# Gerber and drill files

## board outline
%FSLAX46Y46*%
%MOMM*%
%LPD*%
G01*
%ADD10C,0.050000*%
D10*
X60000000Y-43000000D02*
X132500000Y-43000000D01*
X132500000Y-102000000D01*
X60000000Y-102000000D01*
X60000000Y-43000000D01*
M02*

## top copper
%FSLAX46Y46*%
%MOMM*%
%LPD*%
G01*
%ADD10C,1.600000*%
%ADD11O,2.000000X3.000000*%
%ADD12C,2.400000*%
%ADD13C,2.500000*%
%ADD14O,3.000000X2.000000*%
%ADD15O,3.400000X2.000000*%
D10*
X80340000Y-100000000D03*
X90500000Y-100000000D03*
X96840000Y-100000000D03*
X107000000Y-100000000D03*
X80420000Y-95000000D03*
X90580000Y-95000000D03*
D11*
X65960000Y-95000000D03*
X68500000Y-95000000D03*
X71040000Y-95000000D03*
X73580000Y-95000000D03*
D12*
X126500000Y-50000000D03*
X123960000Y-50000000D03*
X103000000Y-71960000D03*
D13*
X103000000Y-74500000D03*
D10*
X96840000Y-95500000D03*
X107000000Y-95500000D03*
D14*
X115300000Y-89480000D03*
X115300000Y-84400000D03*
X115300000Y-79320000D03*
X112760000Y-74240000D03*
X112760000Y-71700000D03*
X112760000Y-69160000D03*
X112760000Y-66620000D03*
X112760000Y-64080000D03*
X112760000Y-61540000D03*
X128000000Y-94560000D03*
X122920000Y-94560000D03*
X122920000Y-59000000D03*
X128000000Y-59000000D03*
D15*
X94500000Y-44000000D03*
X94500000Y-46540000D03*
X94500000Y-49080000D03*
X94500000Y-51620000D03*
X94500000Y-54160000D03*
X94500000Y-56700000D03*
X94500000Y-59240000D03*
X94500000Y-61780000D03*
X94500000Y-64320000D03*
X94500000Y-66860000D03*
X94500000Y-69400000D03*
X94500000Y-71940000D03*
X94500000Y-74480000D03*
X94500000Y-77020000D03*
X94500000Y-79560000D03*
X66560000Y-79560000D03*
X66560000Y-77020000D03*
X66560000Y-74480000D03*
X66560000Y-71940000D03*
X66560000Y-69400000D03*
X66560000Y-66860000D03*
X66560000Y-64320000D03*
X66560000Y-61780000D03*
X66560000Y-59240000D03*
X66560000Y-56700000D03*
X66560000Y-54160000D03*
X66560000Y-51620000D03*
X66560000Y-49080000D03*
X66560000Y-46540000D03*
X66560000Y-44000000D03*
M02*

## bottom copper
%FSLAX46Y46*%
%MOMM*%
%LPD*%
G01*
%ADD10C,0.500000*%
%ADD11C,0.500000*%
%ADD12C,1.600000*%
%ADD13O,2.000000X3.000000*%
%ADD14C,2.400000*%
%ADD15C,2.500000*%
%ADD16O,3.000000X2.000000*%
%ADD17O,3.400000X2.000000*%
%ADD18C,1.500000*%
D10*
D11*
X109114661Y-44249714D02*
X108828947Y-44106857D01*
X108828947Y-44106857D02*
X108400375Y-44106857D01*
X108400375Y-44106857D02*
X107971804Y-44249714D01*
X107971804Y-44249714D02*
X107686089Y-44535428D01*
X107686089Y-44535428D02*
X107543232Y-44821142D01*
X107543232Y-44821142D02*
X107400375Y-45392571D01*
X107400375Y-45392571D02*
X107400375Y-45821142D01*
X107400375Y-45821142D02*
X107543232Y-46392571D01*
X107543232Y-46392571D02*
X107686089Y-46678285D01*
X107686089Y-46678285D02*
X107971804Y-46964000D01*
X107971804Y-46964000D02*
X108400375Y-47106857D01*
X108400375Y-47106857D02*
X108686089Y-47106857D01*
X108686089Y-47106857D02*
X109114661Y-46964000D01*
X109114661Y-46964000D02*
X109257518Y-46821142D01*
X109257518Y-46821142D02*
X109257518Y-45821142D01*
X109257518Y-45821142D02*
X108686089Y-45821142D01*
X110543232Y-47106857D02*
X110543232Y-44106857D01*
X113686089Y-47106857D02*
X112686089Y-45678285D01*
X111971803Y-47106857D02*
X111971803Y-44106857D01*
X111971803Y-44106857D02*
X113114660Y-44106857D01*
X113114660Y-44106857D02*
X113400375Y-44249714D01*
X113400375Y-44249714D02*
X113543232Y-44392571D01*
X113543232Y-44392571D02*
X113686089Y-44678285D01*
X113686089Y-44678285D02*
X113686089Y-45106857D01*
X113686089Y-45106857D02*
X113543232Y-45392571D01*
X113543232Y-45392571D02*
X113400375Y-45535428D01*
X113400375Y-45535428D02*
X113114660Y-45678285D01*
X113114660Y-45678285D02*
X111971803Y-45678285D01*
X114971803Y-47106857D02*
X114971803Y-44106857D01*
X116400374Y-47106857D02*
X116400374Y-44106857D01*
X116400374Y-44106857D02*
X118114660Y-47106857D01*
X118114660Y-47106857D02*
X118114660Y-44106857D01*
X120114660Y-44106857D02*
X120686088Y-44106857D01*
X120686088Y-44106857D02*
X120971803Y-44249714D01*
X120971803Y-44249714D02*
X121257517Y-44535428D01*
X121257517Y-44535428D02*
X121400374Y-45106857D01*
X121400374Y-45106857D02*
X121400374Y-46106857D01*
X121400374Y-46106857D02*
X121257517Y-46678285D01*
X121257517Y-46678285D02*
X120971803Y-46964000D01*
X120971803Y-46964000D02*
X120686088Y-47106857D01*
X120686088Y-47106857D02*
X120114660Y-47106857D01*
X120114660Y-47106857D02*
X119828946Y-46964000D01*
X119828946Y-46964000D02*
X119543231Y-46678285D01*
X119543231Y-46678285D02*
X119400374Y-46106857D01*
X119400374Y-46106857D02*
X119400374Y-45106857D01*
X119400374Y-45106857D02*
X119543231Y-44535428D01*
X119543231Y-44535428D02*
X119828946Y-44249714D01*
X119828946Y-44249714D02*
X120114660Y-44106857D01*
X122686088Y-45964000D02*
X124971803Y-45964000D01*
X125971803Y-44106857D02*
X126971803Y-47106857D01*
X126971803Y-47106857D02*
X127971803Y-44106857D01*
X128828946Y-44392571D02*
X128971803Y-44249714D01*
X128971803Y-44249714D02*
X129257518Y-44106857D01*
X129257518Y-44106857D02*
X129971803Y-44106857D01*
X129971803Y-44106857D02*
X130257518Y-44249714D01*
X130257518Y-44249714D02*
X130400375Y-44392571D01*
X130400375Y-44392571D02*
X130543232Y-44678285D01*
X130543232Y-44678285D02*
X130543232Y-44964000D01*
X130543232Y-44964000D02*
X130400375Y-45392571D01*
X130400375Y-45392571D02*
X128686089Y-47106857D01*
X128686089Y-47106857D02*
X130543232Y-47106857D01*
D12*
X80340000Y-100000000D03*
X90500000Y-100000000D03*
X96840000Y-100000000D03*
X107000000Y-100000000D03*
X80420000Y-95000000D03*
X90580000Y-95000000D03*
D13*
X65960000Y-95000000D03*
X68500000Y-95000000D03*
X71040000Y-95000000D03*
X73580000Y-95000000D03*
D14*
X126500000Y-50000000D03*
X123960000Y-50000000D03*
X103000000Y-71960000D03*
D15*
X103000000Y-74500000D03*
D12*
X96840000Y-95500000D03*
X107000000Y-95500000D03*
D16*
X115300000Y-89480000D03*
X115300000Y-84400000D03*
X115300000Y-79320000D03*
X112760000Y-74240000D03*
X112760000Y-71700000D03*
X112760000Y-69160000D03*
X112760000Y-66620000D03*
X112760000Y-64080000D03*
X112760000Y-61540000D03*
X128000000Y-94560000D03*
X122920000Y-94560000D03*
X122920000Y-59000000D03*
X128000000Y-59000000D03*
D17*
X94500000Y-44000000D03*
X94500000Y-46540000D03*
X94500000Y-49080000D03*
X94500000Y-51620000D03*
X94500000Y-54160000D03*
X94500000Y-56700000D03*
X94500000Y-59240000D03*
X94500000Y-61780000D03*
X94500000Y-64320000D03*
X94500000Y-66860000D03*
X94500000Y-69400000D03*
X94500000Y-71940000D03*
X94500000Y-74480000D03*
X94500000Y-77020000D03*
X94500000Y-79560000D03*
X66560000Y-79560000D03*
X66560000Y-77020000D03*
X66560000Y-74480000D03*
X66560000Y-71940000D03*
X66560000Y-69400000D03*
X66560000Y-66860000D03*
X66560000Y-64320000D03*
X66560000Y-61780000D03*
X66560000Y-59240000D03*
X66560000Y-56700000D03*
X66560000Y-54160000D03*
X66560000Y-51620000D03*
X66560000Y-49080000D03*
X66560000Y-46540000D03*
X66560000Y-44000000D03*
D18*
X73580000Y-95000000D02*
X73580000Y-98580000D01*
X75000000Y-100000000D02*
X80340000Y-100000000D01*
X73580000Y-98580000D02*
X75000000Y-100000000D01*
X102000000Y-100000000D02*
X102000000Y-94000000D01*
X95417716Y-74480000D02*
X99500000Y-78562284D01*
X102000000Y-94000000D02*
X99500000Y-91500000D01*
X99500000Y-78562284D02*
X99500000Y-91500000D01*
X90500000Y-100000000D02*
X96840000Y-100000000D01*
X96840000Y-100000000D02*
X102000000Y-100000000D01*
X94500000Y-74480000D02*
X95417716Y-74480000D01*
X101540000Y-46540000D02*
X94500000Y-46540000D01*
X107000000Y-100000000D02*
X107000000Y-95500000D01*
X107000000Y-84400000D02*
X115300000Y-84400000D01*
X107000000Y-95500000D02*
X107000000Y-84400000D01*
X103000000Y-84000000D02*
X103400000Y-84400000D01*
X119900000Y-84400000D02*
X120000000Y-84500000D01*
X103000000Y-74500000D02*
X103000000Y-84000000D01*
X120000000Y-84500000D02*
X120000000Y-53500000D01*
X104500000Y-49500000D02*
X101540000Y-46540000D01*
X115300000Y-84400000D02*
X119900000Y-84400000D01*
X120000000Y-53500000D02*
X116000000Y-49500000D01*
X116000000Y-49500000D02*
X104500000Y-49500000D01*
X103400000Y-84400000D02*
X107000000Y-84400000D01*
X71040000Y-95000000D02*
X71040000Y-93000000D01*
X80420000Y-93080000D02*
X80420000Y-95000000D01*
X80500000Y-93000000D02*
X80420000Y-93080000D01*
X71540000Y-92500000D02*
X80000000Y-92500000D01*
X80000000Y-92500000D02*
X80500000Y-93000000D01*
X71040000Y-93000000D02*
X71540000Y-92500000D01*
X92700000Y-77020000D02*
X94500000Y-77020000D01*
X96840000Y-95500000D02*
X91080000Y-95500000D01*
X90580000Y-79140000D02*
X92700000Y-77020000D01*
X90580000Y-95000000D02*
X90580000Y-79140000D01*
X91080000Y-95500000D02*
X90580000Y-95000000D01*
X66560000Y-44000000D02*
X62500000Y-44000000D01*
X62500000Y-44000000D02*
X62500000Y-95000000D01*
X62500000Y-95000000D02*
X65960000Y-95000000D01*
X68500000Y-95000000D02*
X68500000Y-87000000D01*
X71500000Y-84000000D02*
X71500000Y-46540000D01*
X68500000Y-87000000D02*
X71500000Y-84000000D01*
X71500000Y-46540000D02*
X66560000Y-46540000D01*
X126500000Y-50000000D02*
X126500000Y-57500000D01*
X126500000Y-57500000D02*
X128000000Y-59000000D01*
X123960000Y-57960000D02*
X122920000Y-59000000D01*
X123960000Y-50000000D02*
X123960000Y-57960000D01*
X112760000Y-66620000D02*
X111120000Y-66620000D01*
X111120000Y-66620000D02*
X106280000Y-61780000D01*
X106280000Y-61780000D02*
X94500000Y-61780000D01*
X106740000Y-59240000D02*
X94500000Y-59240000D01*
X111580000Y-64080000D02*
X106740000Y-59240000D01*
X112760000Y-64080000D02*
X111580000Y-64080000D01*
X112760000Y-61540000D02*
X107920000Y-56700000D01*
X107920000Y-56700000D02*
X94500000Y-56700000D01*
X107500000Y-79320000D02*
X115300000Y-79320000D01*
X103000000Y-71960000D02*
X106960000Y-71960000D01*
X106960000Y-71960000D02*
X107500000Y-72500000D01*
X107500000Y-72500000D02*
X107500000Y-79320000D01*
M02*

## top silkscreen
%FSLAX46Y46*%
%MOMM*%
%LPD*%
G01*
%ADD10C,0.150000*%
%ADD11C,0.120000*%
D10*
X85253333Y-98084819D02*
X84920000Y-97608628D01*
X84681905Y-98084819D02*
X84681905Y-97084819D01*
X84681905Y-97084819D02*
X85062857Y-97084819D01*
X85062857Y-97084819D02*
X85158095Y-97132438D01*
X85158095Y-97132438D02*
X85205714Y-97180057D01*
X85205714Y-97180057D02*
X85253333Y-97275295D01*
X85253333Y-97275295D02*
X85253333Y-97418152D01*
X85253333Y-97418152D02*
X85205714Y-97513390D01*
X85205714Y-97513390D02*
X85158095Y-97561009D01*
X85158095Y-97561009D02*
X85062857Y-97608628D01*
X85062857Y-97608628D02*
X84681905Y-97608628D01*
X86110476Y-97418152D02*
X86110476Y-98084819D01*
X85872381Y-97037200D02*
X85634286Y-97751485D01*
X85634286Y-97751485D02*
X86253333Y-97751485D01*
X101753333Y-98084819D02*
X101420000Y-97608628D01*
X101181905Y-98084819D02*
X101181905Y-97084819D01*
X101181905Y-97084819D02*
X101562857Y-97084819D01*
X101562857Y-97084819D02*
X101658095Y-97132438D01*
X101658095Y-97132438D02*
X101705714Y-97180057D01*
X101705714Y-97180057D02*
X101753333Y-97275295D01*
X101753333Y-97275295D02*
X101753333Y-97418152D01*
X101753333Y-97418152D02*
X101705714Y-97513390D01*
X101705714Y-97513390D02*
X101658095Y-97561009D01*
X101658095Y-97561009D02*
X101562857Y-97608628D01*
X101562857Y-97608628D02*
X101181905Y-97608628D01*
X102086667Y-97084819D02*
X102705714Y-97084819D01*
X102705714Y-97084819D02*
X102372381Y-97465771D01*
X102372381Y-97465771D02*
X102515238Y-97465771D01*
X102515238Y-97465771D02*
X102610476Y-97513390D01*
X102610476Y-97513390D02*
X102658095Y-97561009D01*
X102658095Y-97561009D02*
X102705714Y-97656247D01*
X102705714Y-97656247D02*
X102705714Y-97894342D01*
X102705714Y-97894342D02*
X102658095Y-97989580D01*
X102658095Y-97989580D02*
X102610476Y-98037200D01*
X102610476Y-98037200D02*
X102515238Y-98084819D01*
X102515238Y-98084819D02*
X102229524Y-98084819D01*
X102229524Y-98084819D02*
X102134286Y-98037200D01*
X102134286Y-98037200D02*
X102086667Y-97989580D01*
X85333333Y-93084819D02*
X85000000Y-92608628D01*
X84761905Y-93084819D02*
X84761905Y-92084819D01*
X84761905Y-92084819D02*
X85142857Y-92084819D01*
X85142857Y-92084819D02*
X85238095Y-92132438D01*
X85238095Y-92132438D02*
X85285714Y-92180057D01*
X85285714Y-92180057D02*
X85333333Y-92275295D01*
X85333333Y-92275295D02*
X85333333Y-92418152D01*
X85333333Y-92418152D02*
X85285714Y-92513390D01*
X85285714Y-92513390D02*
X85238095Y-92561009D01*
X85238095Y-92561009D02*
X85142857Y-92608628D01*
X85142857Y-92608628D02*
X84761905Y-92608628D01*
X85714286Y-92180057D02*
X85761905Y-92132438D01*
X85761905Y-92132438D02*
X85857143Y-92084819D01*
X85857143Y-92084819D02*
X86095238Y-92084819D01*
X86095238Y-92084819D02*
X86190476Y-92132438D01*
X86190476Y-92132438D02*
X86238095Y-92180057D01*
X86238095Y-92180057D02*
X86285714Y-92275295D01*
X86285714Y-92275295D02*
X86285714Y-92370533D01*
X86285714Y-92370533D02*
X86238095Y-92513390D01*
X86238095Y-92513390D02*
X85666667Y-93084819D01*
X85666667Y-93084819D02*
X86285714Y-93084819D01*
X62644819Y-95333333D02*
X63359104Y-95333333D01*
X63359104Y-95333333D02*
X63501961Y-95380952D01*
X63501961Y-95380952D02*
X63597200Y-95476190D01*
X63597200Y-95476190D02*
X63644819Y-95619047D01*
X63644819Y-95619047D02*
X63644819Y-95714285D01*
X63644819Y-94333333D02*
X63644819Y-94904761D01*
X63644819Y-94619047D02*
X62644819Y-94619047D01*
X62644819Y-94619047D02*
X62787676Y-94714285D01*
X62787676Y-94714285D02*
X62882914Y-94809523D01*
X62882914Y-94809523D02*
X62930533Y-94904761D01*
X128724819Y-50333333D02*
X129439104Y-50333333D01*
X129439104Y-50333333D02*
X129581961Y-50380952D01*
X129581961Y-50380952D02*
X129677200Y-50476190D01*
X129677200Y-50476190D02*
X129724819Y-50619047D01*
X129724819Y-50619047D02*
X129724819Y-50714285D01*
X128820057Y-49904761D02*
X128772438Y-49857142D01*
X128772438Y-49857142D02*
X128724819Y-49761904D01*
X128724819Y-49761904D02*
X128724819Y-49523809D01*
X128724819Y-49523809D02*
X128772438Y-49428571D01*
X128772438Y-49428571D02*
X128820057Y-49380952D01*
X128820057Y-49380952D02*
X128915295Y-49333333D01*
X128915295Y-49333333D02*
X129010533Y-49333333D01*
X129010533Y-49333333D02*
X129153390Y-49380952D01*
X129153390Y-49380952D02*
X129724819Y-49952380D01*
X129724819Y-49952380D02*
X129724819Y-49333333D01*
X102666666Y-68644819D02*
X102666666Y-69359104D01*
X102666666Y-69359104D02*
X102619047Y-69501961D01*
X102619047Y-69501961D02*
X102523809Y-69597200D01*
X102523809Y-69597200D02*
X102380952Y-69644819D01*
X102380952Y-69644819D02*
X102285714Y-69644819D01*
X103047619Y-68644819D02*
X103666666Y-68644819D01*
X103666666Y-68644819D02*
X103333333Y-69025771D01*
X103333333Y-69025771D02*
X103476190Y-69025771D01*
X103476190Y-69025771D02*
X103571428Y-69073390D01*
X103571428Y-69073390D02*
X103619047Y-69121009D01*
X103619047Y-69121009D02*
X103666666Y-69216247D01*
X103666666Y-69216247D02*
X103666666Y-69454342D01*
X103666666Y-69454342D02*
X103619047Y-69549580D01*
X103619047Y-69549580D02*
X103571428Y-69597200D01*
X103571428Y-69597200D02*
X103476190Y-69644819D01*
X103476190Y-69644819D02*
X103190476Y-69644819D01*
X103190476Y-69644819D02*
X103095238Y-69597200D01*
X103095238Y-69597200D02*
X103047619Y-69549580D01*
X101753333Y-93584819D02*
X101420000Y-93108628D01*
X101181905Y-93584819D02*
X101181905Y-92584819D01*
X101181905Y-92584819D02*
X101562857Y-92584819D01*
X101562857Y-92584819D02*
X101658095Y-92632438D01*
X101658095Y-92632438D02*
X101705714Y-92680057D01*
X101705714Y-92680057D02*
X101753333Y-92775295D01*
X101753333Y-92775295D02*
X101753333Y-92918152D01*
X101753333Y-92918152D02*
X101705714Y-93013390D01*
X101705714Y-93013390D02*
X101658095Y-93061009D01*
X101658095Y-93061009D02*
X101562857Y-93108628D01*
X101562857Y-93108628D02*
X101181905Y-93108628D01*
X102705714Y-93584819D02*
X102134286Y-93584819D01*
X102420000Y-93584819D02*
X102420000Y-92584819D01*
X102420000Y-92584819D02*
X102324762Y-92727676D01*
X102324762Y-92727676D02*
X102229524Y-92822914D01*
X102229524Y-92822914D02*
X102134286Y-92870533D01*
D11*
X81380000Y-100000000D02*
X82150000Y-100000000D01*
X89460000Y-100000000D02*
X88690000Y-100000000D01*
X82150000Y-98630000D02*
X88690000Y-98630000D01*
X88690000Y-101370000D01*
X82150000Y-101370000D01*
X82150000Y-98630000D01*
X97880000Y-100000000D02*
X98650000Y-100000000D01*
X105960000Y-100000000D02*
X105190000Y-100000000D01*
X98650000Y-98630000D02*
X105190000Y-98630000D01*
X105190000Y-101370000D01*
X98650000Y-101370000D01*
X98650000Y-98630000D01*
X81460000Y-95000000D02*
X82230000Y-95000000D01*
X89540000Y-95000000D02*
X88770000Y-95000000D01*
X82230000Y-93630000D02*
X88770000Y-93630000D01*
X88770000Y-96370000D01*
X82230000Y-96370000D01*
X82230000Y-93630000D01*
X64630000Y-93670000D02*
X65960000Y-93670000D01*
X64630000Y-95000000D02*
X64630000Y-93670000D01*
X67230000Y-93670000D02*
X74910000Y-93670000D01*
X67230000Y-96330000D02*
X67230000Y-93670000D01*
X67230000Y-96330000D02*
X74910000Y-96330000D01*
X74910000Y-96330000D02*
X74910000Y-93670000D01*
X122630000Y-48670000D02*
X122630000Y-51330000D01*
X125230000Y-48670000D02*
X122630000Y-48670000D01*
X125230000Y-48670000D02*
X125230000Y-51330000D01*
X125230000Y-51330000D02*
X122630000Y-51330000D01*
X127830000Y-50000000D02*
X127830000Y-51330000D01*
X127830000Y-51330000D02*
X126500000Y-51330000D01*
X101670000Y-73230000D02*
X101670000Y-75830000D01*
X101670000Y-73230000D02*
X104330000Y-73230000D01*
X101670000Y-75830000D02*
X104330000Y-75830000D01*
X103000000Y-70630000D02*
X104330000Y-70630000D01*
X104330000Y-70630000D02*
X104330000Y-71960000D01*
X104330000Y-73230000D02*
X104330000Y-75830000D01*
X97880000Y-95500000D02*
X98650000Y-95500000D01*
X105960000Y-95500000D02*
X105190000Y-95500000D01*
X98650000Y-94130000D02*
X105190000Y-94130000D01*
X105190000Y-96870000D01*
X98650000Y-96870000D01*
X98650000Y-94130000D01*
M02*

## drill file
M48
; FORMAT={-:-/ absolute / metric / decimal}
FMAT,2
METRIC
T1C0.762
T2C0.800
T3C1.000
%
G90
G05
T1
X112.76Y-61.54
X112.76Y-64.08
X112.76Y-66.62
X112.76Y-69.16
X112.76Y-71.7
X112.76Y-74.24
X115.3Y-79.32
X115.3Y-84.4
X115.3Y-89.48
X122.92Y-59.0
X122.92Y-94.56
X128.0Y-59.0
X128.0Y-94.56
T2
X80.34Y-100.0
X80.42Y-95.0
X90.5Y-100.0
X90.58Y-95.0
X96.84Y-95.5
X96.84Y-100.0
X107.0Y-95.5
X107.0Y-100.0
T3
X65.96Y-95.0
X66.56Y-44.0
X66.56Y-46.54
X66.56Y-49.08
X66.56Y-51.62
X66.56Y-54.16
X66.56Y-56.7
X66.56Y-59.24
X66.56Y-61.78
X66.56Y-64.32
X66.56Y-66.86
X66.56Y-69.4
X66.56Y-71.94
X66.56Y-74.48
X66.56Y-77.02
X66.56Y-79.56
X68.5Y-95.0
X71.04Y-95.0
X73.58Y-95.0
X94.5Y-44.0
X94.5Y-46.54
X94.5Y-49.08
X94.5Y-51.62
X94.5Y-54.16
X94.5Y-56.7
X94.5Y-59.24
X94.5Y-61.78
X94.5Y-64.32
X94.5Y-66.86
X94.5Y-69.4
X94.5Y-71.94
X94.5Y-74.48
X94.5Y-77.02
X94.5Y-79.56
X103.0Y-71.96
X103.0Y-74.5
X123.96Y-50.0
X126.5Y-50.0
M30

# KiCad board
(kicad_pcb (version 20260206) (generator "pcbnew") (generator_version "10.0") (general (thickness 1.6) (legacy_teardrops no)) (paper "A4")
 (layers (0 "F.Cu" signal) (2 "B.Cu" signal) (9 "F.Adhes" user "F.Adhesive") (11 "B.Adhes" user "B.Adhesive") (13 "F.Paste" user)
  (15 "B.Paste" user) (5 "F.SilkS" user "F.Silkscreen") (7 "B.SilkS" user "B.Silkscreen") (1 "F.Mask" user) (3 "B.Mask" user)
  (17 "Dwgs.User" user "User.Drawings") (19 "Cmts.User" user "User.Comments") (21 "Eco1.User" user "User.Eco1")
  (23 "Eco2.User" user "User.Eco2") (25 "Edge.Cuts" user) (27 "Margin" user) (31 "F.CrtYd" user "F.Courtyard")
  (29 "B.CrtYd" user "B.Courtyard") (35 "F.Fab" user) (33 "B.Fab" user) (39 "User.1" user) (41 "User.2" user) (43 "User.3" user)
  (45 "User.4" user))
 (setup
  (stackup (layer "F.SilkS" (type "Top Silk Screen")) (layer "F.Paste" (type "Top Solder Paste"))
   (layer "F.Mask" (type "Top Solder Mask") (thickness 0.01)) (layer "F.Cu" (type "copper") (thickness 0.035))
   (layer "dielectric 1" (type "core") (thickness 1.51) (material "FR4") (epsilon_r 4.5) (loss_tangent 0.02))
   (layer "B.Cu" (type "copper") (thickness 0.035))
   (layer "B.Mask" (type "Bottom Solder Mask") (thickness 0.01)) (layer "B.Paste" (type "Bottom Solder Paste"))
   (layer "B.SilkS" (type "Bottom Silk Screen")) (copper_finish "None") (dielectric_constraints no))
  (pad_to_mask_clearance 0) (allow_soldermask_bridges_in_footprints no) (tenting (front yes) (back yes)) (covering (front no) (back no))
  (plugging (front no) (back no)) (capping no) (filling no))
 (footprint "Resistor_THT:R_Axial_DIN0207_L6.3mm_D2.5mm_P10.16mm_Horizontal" (layer "F.Cu") (at 80.34 100)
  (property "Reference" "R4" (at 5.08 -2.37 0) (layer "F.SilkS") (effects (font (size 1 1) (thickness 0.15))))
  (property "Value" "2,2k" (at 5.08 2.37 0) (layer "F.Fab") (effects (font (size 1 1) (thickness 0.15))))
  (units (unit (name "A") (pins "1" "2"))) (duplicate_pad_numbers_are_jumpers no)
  (fp_line (start 1.04 0) (end 1.81 0) (stroke (width 0.12) (type solid)) (layer "F.SilkS"))
  (fp_line (start 9.12 0) (end 8.35 0) (stroke (width 0.12) (type solid)) (layer "F.SilkS"))
  (fp_rect (start 1.81 -1.37) (end 8.35 1.37) (stroke (width 0.12) (type solid)) (fill no) (layer "F.SilkS"))
  (pad "1" thru_hole circle (at 0 0) (size 1.6 1.6) (drill 0.8) (layers "*.Cu" "*.Mask") (remove_unused_layers no) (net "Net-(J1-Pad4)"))
  (pad "2" thru_hole circle (at 10.16 0) (size 1.6 1.6) (drill 0.8) (layers "*.Cu" "*.Mask") (remove_unused_layers no)
   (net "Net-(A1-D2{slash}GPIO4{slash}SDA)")))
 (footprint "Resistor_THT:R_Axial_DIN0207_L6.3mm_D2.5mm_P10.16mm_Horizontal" (layer "F.Cu") (at 96.84 100)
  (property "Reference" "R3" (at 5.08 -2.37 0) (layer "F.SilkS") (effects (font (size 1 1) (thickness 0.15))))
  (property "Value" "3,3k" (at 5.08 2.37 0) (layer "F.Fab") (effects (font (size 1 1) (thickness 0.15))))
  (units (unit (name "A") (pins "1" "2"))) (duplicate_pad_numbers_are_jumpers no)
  (fp_line (start 1.04 0) (end 1.81 0) (stroke (width 0.12) (type solid)) (layer "F.SilkS"))
  (fp_line (start 9.12 0) (end 8.35 0) (stroke (width 0.12) (type solid)) (layer "F.SilkS"))
  (fp_rect (start 1.81 -1.37) (end 8.35 1.37) (stroke (width 0.12) (type solid)) (fill no) (layer "F.SilkS"))
  (pad "1" thru_hole circle (at 0 0) (size 1.6 1.6) (drill 0.8) (layers "*.Cu" "*.Mask") (remove_unused_layers no)
   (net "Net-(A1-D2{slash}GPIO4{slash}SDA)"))
  (pad "2" thru_hole circle (at 10.16 0) (size 1.6 1.6) (drill 0.8) (layers "*.Cu" "*.Mask") (remove_unused_layers no) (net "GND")))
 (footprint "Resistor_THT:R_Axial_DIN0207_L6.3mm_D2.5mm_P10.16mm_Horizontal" (layer "F.Cu") (at 80.42 95)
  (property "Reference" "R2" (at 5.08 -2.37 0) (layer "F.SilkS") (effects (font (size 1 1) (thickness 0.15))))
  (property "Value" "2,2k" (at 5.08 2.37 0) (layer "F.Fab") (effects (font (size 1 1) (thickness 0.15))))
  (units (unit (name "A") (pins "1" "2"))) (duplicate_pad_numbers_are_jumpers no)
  (fp_line (start 1.04 0) (end 1.81 0) (stroke (width 0.12) (type solid)) (layer "F.SilkS"))
  (fp_line (start 9.12 0) (end 8.35 0) (stroke (width 0.12) (type solid)) (layer "F.SilkS"))
  (fp_rect (start 1.81 -1.37) (end 8.35 1.37) (stroke (width 0.12) (type solid)) (fill no) (layer "F.SilkS"))
  (pad "1" thru_hole circle (at 0 0) (size 1.6 1.6) (drill 0.8) (layers "*.Cu" "*.Mask") (remove_unused_layers no) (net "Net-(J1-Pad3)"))
  (pad "2" thru_hole circle (at 10.16 0) (size 1.6 1.6) (drill 0.8) (layers "*.Cu" "*.Mask") (remove_unused_layers no)
   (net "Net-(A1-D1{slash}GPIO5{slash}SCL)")))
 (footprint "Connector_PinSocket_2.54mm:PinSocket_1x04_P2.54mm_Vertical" (layer "F.Cu") (at 65.96 95 90)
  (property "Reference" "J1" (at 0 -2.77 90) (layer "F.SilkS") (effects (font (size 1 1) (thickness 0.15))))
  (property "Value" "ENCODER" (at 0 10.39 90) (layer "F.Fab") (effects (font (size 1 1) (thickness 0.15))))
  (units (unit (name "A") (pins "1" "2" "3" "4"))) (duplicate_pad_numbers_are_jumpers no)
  (fp_line (start 1.33 -1.33) (end 1.33 0) (stroke (width 0.12) (type solid)) (layer "F.SilkS"))
  (fp_line (start 0 -1.33) (end 1.33 -1.33) (stroke (width 0.12) (type solid)) (layer "F.SilkS"))
  (fp_line (start 1.33 1.27) (end 1.33 8.95) (stroke (width 0.12) (type solid)) (layer "F.SilkS"))
  (fp_line (start -1.33 1.27) (end 1.33 1.27) (stroke (width 0.12) (type solid)) (layer "F.SilkS"))
  (fp_line (start -1.33 1.27) (end -1.33 8.95) (stroke (width 0.12) (type solid)) (layer "F.SilkS"))
  (fp_line (start -1.33 8.95) (end 1.33 8.95) (stroke (width 0.12) (type solid)) (layer "F.SilkS"))
  (pad "1" thru_hole oval (at 0 0 90) (size 3 2) (drill 1) (layers "*.Cu" "*.Mask") (remove_unused_layers no) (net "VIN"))
  (pad "2" thru_hole oval (at 0 2.54 90) (size 3 2) (drill 1) (layers "*.Cu" "*.Mask") (remove_unused_layers no) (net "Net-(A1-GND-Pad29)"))
  (pad "3" thru_hole oval (at 0 5.08 90) (size 3 2) (drill 1) (layers "*.Cu" "*.Mask") (remove_unused_layers no) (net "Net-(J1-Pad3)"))
  (pad "4" thru_hole oval (at 0 7.62 90) (size 3 2) (drill 1) (layers "*.Cu" "*.Mask") (remove_unused_layers no) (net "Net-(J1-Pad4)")))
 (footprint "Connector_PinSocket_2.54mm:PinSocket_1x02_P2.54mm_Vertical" (layer "F.Cu") (at 126.5 50 -90)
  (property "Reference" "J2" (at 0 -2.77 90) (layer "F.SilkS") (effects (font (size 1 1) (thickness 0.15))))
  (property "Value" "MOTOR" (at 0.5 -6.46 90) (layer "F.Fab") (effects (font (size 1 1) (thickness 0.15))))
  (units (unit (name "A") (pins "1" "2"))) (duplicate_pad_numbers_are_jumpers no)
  (fp_line (start -1.33 3.87) (end 1.33 3.87) (stroke (width 0.12) (type solid)) (layer "F.SilkS"))
  (fp_line (start -1.33 1.27) (end -1.33 3.87) (stroke (width 0.12) (type solid)) (layer "F.SilkS"))
  (fp_line (start -1.33 1.27) (end 1.33 1.27) (stroke (width 0.12) (type solid)) (layer "F.SilkS"))
  (fp_line (start 1.33 1.27) (end 1.33 3.87) (stroke (width 0.12) (type solid)) (layer "F.SilkS"))
  (fp_line (start 0 -1.33) (end 1.33 -1.33) (stroke (width 0.12) (type solid)) (layer "F.SilkS"))
  (fp_line (start 1.33 -1.33) (end 1.33 0) (stroke (width 0.12) (type solid)) (layer "F.SilkS"))
  (pad "1" thru_hole circle (at 0 0 270) (size 2.4 2.4) (drill 1) (layers "*.Cu" "*.Mask") (remove_unused_layers no) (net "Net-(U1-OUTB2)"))
  (pad "2" thru_hole circle (at 0 2.54 270) (size 2.4 2.4) (drill 1) (layers "*.Cu" "*.Mask") (remove_unused_layers no)
   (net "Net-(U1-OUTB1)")))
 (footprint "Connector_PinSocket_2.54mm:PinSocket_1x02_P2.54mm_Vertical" (layer "F.Cu") (at 103 71.96)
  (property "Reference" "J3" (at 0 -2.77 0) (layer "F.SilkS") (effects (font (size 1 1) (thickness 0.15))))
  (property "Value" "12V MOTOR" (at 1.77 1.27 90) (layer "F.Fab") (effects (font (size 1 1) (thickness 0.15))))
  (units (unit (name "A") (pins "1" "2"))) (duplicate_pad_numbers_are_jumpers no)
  (fp_line (start -1.33 1.27) (end -1.33 3.87) (stroke (width 0.12) (type solid)) (layer "F.SilkS"))
  (fp_line (start -1.33 1.27) (end 1.33 1.27) (stroke (width 0.12) (type solid)) (layer "F.SilkS"))
  (fp_line (start -1.33 3.87) (end 1.33 3.87) (stroke (width 0.12) (type solid)) (layer "F.SilkS"))
  (fp_line (start 0 -1.33) (end 1.33 -1.33) (stroke (width 0.12) (type solid)) (layer "F.SilkS"))
  (fp_line (start 1.33 -1.33) (end 1.33 0) (stroke (width 0.12) (type solid)) (layer "F.SilkS"))
  (fp_line (start 1.33 1.27) (end 1.33 3.87) (stroke (width 0.12) (type solid)) (layer "F.SilkS"))
  (pad "1" thru_hole circle (at 0 0) (size 2.4 2.4) (drill 1) (layers "*.Cu" "*.Mask") (remove_unused_layers no) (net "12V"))
  (pad "2" thru_hole circle (at 0 2.54) (size 2.5 2.5) (drill 1) (layers "*.Cu" "*.Mask") (remove_unused_layers no) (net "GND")))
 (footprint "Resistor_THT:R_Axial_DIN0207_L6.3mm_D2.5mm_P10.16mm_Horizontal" (layer "F.Cu") (at 96.84 95.5)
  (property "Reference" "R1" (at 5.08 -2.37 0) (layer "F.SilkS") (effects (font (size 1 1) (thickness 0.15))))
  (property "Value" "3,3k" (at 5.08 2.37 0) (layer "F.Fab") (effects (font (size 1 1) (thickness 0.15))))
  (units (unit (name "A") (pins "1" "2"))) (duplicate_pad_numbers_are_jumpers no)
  (fp_line (start 1.04 0) (end 1.81 0) (stroke (width 0.12) (type solid)) (layer "F.SilkS"))
  (fp_line (start 9.12 0) (end 8.35 0) (stroke (width 0.12) (type solid)) (layer "F.SilkS"))
  (fp_rect (start 1.81 -1.37) (end 8.35 1.37) (stroke (width 0.12) (type solid)) (fill no) (layer "F.SilkS"))
  (pad "1" thru_hole circle (at 0 0) (size 1.6 1.6) (drill 0.8) (layers "*.Cu" "*.Mask") (remove_unused_layers no)
   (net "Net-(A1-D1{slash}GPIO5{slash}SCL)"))
  (pad "2" thru_hole circle (at 10.16 0) (size 1.6 1.6) (drill 0.8) (layers "*.Cu" "*.Mask") (remove_unused_layers no) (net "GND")))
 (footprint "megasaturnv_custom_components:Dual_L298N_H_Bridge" (layer "B.Cu") (at 110.22 97.1 90)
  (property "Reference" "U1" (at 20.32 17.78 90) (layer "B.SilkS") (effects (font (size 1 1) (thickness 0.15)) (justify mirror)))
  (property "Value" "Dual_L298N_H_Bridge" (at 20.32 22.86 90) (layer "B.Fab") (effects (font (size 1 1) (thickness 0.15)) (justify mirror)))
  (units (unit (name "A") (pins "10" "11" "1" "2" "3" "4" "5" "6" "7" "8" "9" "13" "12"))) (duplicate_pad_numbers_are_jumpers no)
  (pad "1" thru_hole oval (at 7.62 5.08 90) (size 2 3) (drill 0.762) (layers "*.Cu" "*.Mask") (remove_unused_layers no)
   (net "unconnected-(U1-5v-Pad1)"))
  (pad "2" thru_hole oval (at 12.7 5.08 90) (size 2 3) (drill 0.762) (layers "*.Cu" "*.Mask") (remove_unused_layers no) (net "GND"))
  (pad "3" thru_hole oval (at 17.78 5.08 90) (size 2 3) (drill 0.762) (layers "*.Cu" "*.Mask") (remove_unused_layers no) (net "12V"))
  (pad "4" thru_hole oval (at 22.86 2.54 90) (size 2 3) (drill 0.762) (layers "*.Cu" "*.Mask") (remove_unused_layers no)
   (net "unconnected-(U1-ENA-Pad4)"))
  (pad "5" thru_hole oval (at 25.4 2.54 90) (size 2 3) (drill 0.762) (layers "*.Cu" "*.Mask") (remove_unused_layers no)
   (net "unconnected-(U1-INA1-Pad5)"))
  (pad "6" thru_hole oval (at 27.94 2.54 90) (size 2 3) (drill 0.762) (layers "*.Cu" "*.Mask") (remove_unused_layers no)
   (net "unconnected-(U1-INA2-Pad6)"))
  (pad "7" thru_hole oval (at 30.48 2.54 90) (size 2 3) (drill 0.762) (layers "*.Cu" "*.Mask") (remove_unused_layers no)
   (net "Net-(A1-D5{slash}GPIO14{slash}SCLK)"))
  (pad "8" thru_hole oval (at 33.02 2.54 90) (size 2 3) (drill 0.762) (layers "*.Cu" "*.Mask") (remove_unused_layers no)
   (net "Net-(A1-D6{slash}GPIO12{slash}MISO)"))
  (pad "9" thru_hole oval (at 35.56 2.54 90) (size 2 3) (drill 0.762) (layers "*.Cu" "*.Mask") (remove_unused_layers no)
   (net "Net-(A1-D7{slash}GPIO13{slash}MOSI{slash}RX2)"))
  (pad "10" thru_hole oval (at 2.54 17.78 90) (size 2 3) (drill 0.762) (layers "*.Cu" "*.Mask") (remove_unused_layers no)
   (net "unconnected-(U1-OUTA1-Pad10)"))
  (pad "11" thru_hole oval (at 2.54 12.7 90) (size 2 3) (drill 0.762) (layers "*.Cu" "*.Mask") (remove_unused_layers no)
   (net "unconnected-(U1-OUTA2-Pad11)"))
  (pad "12" thru_hole oval (at 38.1 12.7 90) (size 2 3) (drill 0.762) (layers "*.Cu" "*.Mask") (remove_unused_layers no)
   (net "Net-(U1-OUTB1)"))
  (pad "13" thru_hole oval (at 38.1 17.78 90) (size 2 3) (drill 0.762) (layers "*.Cu" "*.Mask") (remove_unused_layers no)
   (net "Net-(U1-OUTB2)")))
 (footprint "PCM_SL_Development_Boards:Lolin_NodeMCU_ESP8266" (layer "B.Cu") (at 80.53 61.78 180)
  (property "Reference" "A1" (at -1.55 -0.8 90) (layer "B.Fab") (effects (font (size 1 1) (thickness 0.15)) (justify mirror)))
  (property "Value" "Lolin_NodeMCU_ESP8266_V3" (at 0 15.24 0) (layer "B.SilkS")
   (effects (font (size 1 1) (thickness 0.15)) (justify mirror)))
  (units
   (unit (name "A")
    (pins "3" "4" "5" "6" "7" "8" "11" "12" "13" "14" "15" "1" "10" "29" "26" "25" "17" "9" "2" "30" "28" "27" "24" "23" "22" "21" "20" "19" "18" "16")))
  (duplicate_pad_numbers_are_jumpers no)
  (pad "1" thru_hole oval (at -13.97 17.78 270) (size 2 3.4) (drill 1) (layers "*.Cu" "*.Mask") (remove_unused_layers no)
   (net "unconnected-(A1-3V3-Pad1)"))
  (pad "2" thru_hole oval (at -13.97 15.24 270) (size 2 3.4) (drill 1) (layers "*.Cu" "*.Mask") (remove_unused_layers no) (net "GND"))
  (pad "3" thru_hole oval (at -13.97 12.7 270) (size 2 3.4) (drill 1) (layers "*.Cu" "*.Mask") (remove_unused_layers no)
   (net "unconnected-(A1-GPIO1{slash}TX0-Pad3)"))
  (pad "4" thru_hole oval (at -13.97 10.16 270) (size 2 3.4) (drill 1) (layers "*.Cu" "*.Mask") (remove_unused_layers no)
   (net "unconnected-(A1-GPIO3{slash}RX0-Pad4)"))
  (pad "5" thru_hole oval (at -13.97 7.62 270) (size 2 3.4) (drill 1) (layers "*.Cu" "*.Mask") (remove_unused_layers no)
   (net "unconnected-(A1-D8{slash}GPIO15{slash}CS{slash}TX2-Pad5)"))
  (pad "6" thru_hole oval (at -13.97 5.08 270) (size 2 3.4) (drill 1) (layers "*.Cu" "*.Mask") (remove_unused_layers no)
   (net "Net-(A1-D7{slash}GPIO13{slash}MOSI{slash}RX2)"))
  (pad "7" thru_hole oval (at -13.97 2.54 270) (size 2 3.4) (drill 1) (layers "*.Cu" "*.Mask") (remove_unused_layers no)
   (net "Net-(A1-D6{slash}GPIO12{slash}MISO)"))
  (pad "8" thru_hole oval (at -13.97 0 270) (size 2 3.4) (drill 1) (layers "*.Cu" "*.Mask") (remove_unused_layers no)
   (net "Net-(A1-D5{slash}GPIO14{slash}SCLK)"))
  (pad "9" thru_hole oval (at -13.97 -2.54 270) (size 2 3.4) (drill 1) (layers "*.Cu" "*.Mask") (remove_unused_layers no)
   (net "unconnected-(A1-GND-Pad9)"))
  (pad "10" thru_hole oval (at -13.97 -5.08 270) (size 2 3.4) (drill 1) (layers "*.Cu" "*.Mask") (remove_unused_layers no)
   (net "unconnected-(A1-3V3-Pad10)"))
  (pad "11" thru_hole oval (at -13.97 -7.62 270) (size 2 3.4) (drill 1) (layers "*.Cu" "*.Mask") (remove_unused_layers no)
   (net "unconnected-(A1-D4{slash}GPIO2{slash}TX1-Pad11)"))
  (pad "12" thru_hole oval (at -13.97 -10.16 270) (size 2 3.4) (drill 1) (layers "*.Cu" "*.Mask") (remove_unused_layers no)
   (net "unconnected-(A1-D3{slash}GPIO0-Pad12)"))
  (pad "13" thru_hole oval (at -13.97 -12.7 270) (size 2 3.4) (drill 1) (layers "*.Cu" "*.Mask") (remove_unused_layers no)
   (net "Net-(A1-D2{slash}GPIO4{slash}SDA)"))
  (pad "14" thru_hole oval (at -13.97 -15.24 270) (size 2 3.4) (drill 1) (layers "*.Cu" "*.Mask") (remove_unused_layers no)
   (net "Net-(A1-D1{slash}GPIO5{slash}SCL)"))
  (pad "15" thru_hole oval (at -13.97 -17.78 270) (size 2 3.4) (drill 1) (layers "*.Cu" "*.Mask") (remove_unused_layers no)
   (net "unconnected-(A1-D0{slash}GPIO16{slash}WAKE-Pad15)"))
  (pad "16" thru_hole oval (at 13.97 -17.78 270) (size 2 3.4) (drill 1) (layers "*.Cu" "*.Mask") (remove_unused_layers no)
   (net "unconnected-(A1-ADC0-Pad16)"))
  (pad "17" thru_hole oval (at 13.97 -15.24 270) (size 2 3.4) (drill 1) (layers "*.Cu" "*.Mask") (remove_unused_layers no)
   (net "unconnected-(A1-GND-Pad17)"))
  (pad "18" thru_hole oval (at 13.97 -12.7 270) (size 2 3.4) (drill 1) (layers "*.Cu" "*.Mask") (remove_unused_layers no)
   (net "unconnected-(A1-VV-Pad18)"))
  (pad "19" thru_hole oval (at 13.97 -10.16 270) (size 2 3.4) (drill 1) (layers "*.Cu" "*.Mask") (remove_unused_layers no)
   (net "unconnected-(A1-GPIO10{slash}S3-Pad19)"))
  (pad "20" thru_hole oval (at 13.97 -7.62 270) (size 2 3.4) (drill 1) (layers "*.Cu" "*.Mask") (remove_unused_layers no)
   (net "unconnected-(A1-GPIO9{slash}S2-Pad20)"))
  (pad "21" thru_hole oval (at 13.97 -5.08 270) (size 2 3.4) (drill 1) (layers "*.Cu" "*.Mask") (remove_unused_layers no)
   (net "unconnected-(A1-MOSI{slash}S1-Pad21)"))
  (pad "22" thru_hole oval (at 13.97 -2.54 270) (size 2 3.4) (drill 1) (layers "*.Cu" "*.Mask") (remove_unused_layers no)
   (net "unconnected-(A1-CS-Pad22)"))
  (pad "23" thru_hole oval (at 13.97 0 270) (size 2 3.4) (drill 1) (layers "*.Cu" "*.Mask") (remove_unused_layers no)
   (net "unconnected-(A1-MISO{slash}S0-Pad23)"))
  (pad "24" thru_hole oval (at 13.97 2.54 270) (size 2 3.4) (drill 1) (layers "*.Cu" "*.Mask") (remove_unused_layers no)
   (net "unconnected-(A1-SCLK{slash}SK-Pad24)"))
  (pad "25" thru_hole oval (at 13.97 5.08 270) (size 2 3.4) (drill 1) (layers "*.Cu" "*.Mask") (remove_unused_layers no)
   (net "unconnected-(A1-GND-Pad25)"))
  (pad "26" thru_hole oval (at 13.97 7.62 270) (size 2 3.4) (drill 1) (layers "*.Cu" "*.Mask") (remove_unused_layers no)
   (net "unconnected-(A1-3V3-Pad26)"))
  (pad "27" thru_hole oval (at 13.97 10.16 270) (size 2 3.4) (drill 1) (layers "*.Cu" "*.Mask") (remove_unused_layers no)
   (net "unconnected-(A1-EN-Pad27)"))
  (pad "28" thru_hole oval (at 13.97 12.7 270) (size 2 3.4) (drill 1) (layers "*.Cu" "*.Mask") (remove_unused_layers no)
   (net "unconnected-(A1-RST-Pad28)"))
  (pad "29" thru_hole oval (at 13.97 15.24 270) (size 2 3.4) (drill 1) (layers "*.Cu" "*.Mask") (remove_unused_layers no)
   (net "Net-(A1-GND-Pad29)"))
  (pad "30" thru_hole oval (at 13.97 17.78 270) (size 2 3.4) (drill 1) (layers "*.Cu" "*.Mask") (remove_unused_layers no) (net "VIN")))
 (gr_rect (start 60 43) (end 132.5 102) (stroke (width 0.05) (type default)) (fill no) (layer "Edge.Cuts"))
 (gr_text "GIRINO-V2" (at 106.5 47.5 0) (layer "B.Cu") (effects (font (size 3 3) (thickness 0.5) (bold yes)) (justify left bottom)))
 (segment (start 73.58 95) (end 73.58 98.58) (width 1.5) (layer "B.Cu") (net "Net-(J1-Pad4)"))
 (segment (start 75 100) (end 80.34 100) (width 1.5) (layer "B.Cu") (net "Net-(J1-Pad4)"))
 (segment (start 73.58 98.58) (end 75 100) (width 1.5) (layer "B.Cu") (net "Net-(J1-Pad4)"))
 (segment (start 102 100) (end 102 94) (width 1.5) (layer "B.Cu") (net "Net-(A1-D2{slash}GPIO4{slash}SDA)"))
 (segment (start 95.417716 74.48) (end 99.5 78.562284) (width 1.5) (layer "B.Cu") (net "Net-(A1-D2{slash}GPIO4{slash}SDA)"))
 (segment (start 102 94) (end 99.5 91.5) (width 1.5) (layer "B.Cu") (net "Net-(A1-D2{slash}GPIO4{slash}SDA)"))
 (segment (start 99.5 78.562284) (end 99.5 91.5) (width 1.5) (layer "B.Cu") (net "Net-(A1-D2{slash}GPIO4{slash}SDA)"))
 (segment (start 90.5 100) (end 96.84 100) (width 1.5) (layer "B.Cu") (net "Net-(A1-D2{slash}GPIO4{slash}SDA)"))
 (segment (start 96.84 100) (end 102 100) (width 1.5) (layer "B.Cu") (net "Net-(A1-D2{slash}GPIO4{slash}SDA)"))
 (segment (start 94.5 74.48) (end 95.417716 74.48) (width 1.5) (layer "B.Cu") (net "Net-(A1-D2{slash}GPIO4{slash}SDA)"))
 (segment (start 101.54 46.54) (end 94.5 46.54) (width 1.5) (layer "B.Cu") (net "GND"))
 (segment (start 107 100) (end 107 95.5) (width 1.5) (layer "B.Cu") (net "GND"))
 (segment (start 107 84.4) (end 115.3 84.4) (width 1.5) (layer "B.Cu") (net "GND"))
 (segment (start 107 95.5) (end 107 84.4) (width 1.5) (layer "B.Cu") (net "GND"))
 (segment (start 103 84) (end 103.4 84.4) (width 1.5) (layer "B.Cu") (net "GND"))
 (segment (start 119.9 84.4) (end 120 84.5) (width 1.5) (layer "B.Cu") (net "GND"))
 (segment (start 103 74.5) (end 103 84) (width 1.5) (layer "B.Cu") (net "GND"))
 (segment (start 120 84.5) (end 120 53.5) (width 1.5) (layer "B.Cu") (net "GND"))
 (segment (start 104.5 49.5) (end 101.54 46.54) (width 1.5) (layer "B.Cu") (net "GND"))
 (segment (start 115.3 84.4) (end 119.9 84.4) (width 1.5) (layer "B.Cu") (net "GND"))
 (segment (start 120 53.5) (end 116 49.5) (width 1.5) (layer "B.Cu") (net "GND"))
 (segment (start 116 49.5) (end 104.5 49.5) (width 1.5) (layer "B.Cu") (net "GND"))
 (segment (start 103.4 84.4) (end 107 84.4) (width 1.5) (layer "B.Cu") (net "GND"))
 (segment (start 71.04 95) (end 71.04 93) (width 1.5) (layer "B.Cu") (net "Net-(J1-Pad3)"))
 (segment (start 80.42 93.08) (end 80.42 95) (width 1.5) (layer "B.Cu") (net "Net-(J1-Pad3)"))
 (segment (start 80.5 93) (end 80.42 93.08) (width 1.5) (layer "B.Cu") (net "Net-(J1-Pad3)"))
 (segment (start 71.54 92.5) (end 80 92.5) (width 1.5) (layer "B.Cu") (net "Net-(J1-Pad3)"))
 (segment (start 80 92.5) (end 80.5 93) (width 1.5) (layer "B.Cu") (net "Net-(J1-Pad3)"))
 (segment (start 71.04 93) (end 71.54 92.5) (width 1.5) (layer "B.Cu") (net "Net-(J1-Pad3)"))
 (segment (start 92.7 77.02) (end 94.5 77.02) (width 1.5) (layer "B.Cu") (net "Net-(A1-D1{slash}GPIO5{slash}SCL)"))
 (segment (start 96.84 95.5) (end 91.08 95.5) (width 1.5) (layer "B.Cu") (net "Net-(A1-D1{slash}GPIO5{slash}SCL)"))
 (segment (start 90.58 79.14) (end 92.7 77.02) (width 1.5) (layer "B.Cu") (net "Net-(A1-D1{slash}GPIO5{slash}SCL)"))
 (segment (start 90.58 95) (end 90.58 79.14) (width 1.5) (layer "B.Cu") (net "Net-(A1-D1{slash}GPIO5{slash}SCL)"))
 (segment (start 91.08 95.5) (end 90.58 95) (width 1.5) (layer "B.Cu") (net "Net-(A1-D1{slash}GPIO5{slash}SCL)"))
 (segment (start 66.56 44) (end 62.5 44) (width 1.5) (layer "B.Cu") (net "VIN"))
 (segment (start 62.5 44) (end 62.5 95) (width 1.5) (layer "B.Cu") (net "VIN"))
 (segment (start 62.5 95) (end 65.96 95) (width 1.5) (layer "B.Cu") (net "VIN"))
 (segment (start 68.5 95) (end 68.5 87) (width 1.5) (layer "B.Cu") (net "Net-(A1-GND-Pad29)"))
 (segment (start 71.5 84) (end 71.5 46.54) (width 1.5) (layer "B.Cu") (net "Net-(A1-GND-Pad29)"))
 (segment (start 68.5 87) (end 71.5 84) (width 1.5) (layer "B.Cu") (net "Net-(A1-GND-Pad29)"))
 (segment (start 71.5 46.54) (end 66.56 46.54) (width 1.5) (layer "B.Cu") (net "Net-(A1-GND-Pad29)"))
 (segment (start 126.5 50) (end 126.5 57.5) (width 1.5) (layer "B.Cu") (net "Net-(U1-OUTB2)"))
 (segment (start 126.5 57.5) (end 128 59) (width 1.5) (layer "B.Cu") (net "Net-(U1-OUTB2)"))
 (segment (start 123.96 57.96) (end 122.92 59) (width 1.5) (layer "B.Cu") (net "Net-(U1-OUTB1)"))
 (segment (start 123.96 50) (end 123.96 57.96) (width 1.5) (layer "B.Cu") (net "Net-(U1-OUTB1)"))
 (segment (start 112.76 66.62) (end 111.12 66.62) (width 1.5) (layer "B.Cu") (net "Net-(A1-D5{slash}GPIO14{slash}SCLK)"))
 (segment (start 111.12 66.62) (end 106.28 61.78) (width 1.5) (layer "B.Cu") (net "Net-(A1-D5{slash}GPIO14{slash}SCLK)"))
 (segment (start 106.28 61.78) (end 94.5 61.78) (width 1.5) (layer "B.Cu") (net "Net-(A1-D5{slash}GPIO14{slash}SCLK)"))
 (segment (start 106.74 59.24) (end 94.5 59.24) (width 1.5) (layer "B.Cu") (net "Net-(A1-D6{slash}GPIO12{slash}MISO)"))
 (segment (start 111.58 64.08) (end 106.74 59.24) (width 1.5) (layer "B.Cu") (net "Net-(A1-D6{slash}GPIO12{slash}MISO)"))
 (segment (start 112.76 64.08) (end 111.58 64.08) (width 1.5) (layer "B.Cu") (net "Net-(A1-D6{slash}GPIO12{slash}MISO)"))
 (segment (start 112.76 61.54) (end 107.92 56.7) (width 1.5) (layer "B.Cu") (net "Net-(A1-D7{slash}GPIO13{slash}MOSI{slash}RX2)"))
 (segment (start 107.92 56.7) (end 94.5 56.7) (width 1.5) (layer "B.Cu") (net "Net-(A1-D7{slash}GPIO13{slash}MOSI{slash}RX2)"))
 (segment (start 107.5 79.32) (end 115.3 79.32) (width 1.5) (layer "B.Cu") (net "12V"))
 (segment (start 103 71.96) (end 106.96 71.96) (width 1.5) (layer "B.Cu") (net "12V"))
 (segment (start 106.96 71.96) (end 107.5 72.5) (width 1.5) (layer "B.Cu") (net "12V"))
 (segment (start 107.5 72.5) (end 107.5 79.32) (width 1.5) (layer "B.Cu") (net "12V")))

